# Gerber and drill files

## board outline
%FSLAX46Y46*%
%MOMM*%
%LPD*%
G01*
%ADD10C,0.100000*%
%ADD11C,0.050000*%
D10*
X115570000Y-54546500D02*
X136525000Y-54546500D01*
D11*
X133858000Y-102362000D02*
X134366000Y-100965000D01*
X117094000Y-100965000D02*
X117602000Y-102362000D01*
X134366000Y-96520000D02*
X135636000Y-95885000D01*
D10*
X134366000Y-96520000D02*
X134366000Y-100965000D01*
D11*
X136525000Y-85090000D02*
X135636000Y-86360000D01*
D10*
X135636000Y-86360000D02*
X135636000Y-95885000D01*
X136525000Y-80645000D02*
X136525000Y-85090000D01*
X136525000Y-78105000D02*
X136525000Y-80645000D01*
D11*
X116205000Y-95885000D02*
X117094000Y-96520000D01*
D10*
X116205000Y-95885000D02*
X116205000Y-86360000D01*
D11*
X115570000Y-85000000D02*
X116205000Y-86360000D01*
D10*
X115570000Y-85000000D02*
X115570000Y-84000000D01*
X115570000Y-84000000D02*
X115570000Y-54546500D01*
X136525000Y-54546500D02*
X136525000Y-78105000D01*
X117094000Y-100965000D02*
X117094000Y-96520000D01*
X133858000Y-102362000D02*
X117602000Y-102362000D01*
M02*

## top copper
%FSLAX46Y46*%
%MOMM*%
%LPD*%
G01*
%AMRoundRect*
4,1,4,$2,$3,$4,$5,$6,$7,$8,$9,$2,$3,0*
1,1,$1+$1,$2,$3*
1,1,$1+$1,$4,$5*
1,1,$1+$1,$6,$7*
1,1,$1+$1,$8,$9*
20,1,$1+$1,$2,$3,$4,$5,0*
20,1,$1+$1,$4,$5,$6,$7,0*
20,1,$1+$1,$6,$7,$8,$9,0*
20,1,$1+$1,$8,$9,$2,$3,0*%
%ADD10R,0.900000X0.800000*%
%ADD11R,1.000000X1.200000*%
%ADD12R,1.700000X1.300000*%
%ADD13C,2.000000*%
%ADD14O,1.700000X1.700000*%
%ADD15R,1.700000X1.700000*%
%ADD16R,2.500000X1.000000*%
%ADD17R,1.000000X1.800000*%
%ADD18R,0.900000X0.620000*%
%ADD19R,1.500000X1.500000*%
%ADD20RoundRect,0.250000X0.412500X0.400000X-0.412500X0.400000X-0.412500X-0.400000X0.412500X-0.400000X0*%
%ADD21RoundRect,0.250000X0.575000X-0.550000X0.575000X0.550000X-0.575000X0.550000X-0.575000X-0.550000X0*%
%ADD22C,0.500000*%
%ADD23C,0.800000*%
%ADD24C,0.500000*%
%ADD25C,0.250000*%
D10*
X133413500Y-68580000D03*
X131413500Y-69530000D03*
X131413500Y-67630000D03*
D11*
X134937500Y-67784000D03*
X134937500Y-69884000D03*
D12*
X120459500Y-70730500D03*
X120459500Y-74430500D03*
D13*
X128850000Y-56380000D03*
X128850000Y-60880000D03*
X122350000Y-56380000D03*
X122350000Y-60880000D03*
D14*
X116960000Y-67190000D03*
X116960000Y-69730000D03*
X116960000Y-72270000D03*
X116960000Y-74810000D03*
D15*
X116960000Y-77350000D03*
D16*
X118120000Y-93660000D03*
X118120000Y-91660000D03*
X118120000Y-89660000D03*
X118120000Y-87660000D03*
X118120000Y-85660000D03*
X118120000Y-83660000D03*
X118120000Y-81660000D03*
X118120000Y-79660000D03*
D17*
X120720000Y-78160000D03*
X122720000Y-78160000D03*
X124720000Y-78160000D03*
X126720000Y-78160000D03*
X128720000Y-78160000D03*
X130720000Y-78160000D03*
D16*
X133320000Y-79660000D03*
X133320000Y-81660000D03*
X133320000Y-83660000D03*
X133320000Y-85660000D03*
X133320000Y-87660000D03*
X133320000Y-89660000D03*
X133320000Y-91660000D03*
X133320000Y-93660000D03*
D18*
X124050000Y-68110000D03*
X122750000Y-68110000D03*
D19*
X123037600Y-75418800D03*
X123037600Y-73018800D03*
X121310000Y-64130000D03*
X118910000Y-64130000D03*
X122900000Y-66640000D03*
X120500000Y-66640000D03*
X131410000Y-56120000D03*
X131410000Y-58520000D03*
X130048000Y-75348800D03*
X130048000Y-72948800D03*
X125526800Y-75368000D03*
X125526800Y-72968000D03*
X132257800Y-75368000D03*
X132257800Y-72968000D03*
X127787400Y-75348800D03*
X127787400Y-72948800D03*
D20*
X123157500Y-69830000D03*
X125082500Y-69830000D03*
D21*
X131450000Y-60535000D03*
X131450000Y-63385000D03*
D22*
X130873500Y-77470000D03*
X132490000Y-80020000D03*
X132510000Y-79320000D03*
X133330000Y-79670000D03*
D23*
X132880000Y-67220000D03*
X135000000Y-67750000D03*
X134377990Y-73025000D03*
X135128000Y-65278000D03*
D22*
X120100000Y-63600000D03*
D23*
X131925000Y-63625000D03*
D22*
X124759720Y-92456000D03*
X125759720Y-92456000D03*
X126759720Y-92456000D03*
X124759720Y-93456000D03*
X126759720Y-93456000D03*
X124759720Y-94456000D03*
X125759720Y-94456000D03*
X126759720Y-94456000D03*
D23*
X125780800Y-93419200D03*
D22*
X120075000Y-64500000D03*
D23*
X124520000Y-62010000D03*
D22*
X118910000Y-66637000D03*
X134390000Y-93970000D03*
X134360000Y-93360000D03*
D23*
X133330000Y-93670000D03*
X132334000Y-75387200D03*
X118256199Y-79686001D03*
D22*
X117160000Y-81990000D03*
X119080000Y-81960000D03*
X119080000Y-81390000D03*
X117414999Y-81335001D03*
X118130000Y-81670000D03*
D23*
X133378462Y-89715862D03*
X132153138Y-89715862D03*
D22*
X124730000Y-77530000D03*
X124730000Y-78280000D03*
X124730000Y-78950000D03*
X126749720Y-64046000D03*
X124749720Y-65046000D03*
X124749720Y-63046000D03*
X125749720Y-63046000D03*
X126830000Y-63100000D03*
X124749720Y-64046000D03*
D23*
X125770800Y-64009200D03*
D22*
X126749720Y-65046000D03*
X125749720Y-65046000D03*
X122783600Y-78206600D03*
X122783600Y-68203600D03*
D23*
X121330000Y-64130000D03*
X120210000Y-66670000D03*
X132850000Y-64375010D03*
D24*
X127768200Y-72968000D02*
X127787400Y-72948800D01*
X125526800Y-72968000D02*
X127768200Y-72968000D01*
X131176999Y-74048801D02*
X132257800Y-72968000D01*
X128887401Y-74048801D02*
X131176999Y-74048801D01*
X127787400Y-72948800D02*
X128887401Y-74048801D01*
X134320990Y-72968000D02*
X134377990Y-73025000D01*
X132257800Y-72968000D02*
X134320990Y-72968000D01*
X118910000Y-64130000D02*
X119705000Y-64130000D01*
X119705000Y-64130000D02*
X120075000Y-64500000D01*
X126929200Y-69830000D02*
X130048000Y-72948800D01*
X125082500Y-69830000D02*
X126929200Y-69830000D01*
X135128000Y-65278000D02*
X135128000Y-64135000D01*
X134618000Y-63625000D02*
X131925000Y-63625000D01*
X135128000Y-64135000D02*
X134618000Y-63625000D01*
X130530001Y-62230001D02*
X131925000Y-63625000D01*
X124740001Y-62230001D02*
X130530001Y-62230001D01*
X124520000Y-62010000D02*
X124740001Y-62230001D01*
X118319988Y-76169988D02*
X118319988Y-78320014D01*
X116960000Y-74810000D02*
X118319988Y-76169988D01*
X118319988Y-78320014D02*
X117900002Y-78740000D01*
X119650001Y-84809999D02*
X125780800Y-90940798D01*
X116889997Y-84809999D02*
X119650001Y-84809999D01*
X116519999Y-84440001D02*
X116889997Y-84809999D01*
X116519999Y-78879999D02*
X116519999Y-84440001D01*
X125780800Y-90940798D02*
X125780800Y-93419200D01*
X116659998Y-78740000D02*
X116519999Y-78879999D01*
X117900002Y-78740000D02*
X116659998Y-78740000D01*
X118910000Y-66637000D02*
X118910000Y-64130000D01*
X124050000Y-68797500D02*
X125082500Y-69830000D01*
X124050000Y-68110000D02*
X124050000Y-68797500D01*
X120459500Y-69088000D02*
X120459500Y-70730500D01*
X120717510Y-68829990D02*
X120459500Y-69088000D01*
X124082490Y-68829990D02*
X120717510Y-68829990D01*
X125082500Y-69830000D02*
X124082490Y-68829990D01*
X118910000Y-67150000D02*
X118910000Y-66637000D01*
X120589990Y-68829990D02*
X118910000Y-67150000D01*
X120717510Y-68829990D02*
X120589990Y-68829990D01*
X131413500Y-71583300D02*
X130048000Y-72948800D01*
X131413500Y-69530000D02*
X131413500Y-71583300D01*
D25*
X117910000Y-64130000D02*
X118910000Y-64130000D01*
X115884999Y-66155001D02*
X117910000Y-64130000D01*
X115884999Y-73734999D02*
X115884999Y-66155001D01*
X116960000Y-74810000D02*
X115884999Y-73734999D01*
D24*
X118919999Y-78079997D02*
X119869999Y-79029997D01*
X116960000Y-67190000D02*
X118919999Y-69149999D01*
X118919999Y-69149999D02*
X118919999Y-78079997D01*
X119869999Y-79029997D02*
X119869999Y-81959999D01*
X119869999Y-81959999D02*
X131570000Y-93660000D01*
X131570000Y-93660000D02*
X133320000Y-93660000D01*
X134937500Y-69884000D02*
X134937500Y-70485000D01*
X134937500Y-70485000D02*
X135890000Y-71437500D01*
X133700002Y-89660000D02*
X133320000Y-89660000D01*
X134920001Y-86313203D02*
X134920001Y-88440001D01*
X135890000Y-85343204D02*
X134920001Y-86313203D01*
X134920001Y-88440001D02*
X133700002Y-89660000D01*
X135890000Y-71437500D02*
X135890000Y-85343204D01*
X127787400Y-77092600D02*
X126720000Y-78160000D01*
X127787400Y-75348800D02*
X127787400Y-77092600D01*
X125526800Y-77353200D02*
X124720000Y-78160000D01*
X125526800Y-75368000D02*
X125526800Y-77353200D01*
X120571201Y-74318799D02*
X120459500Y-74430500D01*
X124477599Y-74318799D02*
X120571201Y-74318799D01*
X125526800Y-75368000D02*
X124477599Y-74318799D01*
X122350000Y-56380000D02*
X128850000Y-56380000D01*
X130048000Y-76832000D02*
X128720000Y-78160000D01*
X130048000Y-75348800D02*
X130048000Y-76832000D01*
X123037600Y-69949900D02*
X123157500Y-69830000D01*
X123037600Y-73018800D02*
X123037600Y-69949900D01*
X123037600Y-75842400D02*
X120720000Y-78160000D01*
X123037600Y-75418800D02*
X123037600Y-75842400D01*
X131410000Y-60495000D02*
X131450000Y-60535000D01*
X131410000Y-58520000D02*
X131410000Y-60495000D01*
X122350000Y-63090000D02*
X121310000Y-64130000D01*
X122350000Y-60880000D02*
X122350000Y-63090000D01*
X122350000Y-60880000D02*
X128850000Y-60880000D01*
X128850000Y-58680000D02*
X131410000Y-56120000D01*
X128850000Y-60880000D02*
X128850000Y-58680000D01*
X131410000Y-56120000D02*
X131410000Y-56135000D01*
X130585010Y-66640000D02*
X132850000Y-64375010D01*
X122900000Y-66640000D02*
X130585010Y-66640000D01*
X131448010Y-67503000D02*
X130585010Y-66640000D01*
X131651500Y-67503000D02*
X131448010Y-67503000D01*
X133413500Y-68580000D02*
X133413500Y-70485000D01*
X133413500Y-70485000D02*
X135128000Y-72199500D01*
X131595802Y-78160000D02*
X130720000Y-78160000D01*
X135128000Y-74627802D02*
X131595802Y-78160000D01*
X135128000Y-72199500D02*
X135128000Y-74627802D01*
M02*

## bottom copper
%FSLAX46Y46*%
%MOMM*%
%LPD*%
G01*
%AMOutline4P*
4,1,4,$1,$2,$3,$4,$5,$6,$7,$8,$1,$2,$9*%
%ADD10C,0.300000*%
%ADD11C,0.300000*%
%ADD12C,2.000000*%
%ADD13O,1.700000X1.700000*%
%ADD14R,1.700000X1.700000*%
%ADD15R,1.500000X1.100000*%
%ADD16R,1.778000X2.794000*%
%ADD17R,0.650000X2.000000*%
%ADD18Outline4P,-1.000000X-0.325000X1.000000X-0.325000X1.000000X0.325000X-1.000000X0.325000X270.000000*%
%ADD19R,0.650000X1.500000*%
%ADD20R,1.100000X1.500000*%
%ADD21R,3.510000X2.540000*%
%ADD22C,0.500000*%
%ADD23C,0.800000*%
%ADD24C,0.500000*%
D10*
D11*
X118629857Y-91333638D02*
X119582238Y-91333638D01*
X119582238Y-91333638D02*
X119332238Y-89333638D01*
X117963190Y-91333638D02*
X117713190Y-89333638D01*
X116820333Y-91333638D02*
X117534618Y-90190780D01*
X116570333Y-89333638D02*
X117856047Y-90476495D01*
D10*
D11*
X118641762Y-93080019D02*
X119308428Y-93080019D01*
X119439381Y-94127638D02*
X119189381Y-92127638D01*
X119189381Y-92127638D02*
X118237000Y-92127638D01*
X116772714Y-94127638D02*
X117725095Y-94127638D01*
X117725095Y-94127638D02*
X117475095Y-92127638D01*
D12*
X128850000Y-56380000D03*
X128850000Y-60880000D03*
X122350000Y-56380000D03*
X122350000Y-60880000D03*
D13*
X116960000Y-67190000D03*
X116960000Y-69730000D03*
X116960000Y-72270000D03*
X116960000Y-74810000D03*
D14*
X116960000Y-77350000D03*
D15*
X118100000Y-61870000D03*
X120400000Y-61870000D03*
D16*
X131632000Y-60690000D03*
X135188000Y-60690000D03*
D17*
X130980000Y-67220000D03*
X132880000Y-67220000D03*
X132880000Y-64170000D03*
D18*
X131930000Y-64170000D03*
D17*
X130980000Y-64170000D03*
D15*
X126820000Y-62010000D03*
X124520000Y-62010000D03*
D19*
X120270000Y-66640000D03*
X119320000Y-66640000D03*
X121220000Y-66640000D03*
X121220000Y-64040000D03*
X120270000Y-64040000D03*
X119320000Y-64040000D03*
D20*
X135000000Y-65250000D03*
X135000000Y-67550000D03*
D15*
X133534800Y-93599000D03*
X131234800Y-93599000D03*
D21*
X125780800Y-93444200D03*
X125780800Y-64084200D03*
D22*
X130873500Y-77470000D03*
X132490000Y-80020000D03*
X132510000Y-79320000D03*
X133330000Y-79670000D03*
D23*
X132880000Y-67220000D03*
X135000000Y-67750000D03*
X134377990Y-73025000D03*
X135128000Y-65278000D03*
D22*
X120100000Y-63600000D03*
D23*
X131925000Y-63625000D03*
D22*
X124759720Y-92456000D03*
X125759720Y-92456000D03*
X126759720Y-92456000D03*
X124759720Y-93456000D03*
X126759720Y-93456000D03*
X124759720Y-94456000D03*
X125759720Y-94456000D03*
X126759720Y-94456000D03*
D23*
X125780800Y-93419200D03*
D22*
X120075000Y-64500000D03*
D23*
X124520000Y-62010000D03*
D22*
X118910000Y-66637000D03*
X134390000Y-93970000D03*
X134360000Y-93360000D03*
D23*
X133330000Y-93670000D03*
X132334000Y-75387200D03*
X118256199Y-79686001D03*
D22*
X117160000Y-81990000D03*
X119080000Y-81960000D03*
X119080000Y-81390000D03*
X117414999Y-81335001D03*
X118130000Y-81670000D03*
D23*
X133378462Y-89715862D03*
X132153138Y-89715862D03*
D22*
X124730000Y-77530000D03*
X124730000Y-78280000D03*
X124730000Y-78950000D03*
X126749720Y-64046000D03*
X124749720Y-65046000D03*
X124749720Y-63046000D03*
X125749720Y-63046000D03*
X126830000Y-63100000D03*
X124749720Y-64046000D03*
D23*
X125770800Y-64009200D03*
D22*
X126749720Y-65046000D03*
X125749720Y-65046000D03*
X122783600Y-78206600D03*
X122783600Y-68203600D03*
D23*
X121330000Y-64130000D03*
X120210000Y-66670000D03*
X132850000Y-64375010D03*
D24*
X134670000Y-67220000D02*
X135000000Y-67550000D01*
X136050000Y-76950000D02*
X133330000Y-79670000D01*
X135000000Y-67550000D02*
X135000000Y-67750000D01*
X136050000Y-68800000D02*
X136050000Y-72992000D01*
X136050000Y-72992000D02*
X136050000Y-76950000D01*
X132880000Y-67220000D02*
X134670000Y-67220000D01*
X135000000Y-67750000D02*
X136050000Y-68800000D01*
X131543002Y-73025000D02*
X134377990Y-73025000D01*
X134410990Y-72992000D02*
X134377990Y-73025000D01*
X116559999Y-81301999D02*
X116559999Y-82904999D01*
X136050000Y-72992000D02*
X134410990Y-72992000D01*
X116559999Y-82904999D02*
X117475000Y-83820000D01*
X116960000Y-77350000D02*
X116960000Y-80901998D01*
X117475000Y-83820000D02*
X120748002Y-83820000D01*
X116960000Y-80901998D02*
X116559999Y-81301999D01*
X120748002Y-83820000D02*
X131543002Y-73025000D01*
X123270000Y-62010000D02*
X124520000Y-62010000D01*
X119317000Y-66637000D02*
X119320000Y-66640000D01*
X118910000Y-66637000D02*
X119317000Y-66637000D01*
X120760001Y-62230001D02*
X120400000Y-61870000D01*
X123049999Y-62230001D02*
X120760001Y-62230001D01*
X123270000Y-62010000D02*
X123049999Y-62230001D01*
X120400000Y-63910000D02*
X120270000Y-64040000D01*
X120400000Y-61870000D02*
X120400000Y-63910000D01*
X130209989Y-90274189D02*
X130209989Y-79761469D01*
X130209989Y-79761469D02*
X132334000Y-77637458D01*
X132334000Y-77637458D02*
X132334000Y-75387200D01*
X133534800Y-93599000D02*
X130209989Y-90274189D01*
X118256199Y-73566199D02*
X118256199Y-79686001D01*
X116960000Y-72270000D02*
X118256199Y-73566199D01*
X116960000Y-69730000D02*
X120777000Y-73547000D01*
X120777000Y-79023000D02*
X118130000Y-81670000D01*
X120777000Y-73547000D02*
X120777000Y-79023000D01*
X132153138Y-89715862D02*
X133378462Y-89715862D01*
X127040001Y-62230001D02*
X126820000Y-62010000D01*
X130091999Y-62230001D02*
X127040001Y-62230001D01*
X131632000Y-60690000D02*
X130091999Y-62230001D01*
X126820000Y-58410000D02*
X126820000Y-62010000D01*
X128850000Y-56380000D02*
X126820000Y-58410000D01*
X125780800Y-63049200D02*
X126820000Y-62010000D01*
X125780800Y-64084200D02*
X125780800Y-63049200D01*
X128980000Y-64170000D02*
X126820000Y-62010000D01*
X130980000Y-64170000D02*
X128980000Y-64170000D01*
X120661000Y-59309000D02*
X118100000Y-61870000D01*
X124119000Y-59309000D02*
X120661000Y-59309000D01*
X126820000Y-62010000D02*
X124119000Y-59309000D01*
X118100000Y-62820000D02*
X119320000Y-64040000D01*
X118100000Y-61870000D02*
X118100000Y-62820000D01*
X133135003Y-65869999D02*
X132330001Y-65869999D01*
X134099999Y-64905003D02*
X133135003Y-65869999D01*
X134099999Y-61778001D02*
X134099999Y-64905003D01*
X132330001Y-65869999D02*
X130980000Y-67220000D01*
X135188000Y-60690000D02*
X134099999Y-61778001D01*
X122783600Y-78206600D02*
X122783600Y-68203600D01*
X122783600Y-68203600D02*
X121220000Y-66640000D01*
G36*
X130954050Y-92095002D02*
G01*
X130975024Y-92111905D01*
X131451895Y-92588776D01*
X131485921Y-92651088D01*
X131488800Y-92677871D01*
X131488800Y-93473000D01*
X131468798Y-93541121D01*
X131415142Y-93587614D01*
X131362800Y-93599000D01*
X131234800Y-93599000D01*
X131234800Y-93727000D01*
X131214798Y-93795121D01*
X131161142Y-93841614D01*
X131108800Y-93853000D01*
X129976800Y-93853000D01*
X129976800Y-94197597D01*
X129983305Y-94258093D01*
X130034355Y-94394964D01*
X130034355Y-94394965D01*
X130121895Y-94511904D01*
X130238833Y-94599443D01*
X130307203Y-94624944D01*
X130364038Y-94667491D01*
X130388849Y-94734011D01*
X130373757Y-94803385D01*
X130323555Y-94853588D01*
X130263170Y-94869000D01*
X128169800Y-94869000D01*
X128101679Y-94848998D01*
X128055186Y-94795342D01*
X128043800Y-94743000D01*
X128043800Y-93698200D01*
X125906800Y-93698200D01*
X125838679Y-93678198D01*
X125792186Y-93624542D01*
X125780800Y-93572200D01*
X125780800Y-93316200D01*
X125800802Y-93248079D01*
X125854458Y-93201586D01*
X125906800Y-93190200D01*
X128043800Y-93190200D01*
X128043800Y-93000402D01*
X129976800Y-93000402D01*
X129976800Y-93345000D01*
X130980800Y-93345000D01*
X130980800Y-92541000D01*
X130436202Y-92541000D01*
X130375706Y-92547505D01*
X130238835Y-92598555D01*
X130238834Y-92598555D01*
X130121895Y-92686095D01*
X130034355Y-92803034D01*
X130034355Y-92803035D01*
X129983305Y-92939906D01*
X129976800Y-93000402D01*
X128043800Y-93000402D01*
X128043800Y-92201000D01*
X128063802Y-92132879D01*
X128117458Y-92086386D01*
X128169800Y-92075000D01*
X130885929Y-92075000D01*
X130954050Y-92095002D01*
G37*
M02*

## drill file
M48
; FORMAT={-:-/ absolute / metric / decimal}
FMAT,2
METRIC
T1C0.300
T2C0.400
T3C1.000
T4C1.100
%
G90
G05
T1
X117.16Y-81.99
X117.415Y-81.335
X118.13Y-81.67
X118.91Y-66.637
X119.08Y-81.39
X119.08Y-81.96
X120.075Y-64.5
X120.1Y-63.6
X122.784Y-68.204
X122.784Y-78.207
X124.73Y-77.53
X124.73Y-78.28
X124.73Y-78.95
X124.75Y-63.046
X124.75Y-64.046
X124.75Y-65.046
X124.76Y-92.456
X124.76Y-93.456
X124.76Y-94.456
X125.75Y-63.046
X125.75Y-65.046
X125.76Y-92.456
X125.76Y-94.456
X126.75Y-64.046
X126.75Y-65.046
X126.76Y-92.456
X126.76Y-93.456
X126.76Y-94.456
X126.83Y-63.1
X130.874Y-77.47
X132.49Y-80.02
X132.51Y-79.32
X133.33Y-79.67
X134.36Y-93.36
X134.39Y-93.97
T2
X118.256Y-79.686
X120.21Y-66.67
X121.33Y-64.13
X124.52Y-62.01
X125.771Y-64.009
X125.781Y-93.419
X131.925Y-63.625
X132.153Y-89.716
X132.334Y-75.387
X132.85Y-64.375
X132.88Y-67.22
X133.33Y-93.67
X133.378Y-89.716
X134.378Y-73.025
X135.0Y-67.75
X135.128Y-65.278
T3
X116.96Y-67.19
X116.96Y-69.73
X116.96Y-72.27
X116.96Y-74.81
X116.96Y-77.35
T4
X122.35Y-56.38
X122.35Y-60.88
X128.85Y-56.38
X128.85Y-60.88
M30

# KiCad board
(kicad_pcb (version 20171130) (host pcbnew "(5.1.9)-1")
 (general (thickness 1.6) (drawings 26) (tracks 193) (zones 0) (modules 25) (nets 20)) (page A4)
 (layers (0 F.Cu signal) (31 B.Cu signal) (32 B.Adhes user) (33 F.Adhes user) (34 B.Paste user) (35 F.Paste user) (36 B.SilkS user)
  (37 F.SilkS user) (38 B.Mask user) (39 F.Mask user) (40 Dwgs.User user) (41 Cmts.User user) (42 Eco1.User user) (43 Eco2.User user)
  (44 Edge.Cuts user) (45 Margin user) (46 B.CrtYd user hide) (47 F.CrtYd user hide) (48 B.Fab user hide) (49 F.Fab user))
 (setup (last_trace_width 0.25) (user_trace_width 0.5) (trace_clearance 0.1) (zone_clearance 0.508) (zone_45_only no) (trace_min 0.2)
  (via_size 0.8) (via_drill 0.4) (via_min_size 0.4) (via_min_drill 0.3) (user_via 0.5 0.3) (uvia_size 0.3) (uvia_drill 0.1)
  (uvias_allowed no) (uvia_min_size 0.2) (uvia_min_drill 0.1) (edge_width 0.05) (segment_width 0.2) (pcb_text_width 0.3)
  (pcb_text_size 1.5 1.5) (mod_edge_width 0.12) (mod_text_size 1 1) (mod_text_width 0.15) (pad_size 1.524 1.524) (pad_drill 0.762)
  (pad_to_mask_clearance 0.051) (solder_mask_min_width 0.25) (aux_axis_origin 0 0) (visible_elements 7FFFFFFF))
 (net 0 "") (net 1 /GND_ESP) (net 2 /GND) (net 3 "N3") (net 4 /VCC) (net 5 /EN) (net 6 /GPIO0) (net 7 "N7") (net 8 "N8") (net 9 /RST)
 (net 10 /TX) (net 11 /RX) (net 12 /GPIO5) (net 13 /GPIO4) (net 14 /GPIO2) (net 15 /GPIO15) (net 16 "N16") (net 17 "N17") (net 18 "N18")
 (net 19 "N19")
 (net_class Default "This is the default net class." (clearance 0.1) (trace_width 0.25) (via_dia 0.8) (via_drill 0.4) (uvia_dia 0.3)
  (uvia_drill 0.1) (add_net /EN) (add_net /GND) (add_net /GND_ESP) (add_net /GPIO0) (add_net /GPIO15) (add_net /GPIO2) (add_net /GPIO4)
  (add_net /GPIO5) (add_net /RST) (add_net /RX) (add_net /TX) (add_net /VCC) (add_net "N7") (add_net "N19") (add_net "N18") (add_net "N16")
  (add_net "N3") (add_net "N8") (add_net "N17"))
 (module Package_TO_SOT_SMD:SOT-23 (layer F.Cu) (at 132.4135 68.58)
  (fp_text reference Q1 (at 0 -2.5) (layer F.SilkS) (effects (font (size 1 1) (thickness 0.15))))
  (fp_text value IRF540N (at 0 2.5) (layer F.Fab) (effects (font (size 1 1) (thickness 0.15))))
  (pad 3 smd rect (at 1 0) (size 0.9 0.8) (layers F.Cu F.Paste F.Mask) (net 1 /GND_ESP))
  (pad 2 smd rect (at -1 0.95) (size 0.9 0.8) (layers F.Cu F.Paste F.Mask) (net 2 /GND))
  (pad 1 smd rect (at -1 -0.95) (size 0.9 0.8) (layers F.Cu F.Paste F.Mask) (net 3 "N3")))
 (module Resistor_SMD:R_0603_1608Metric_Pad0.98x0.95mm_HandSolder (layer F.Cu) (at 134.9375 68.834 90)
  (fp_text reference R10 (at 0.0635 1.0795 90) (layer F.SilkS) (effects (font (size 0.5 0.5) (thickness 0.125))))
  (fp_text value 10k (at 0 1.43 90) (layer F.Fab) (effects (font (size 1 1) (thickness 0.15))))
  (pad 2 smd rect (at 1.05 0 90) (size 1.2 1) (layers F.Cu F.Paste F.Mask) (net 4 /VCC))
  (pad 1 smd rect (at -1.05 0 90) (size 1.2 1) (layers F.Cu F.Paste F.Mask) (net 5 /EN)))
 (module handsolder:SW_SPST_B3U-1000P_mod (layer F.Cu) (at 120.4595 72.5805 90)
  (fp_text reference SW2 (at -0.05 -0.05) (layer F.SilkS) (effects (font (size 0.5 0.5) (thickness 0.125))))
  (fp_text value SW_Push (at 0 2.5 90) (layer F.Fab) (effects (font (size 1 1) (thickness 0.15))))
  (pad 2 smd rect (at 1.85 0 90) (size 1.3 1.7) (layers F.Cu F.Paste F.Mask) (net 2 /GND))
  (pad 1 smd rect (at -1.85 0 90) (size 1.3 1.7) (layers F.Cu F.Paste F.Mask) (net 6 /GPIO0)))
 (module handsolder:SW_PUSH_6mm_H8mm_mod (layer F.Cu) (at 122.35 56.38)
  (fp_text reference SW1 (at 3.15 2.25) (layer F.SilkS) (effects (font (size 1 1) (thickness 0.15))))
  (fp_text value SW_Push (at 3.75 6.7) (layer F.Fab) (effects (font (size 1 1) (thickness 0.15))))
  (pad 1 thru_hole circle (at 6.5 0 90) (size 2 2) (drill 1.1) (layers *.Cu *.Mask) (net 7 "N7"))
  (pad 2 thru_hole circle (at 6.5 4.5 90) (size 2 2) (drill 1.1) (layers *.Cu *.Mask) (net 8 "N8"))
  (pad 1 thru_hole circle (at 0 0 90) (size 2 2) (drill 1.1) (layers *.Cu *.Mask) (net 7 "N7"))
  (pad 2 thru_hole circle (at 0 4.5 90) (size 2 2) (drill 1.1) (layers *.Cu *.Mask) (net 8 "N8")))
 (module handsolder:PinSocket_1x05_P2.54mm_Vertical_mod (layer F.Cu) (at 116.96 77.35 180)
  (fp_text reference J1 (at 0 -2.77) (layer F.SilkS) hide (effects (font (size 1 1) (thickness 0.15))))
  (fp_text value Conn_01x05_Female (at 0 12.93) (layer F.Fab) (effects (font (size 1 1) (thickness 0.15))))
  (pad 5 thru_hole oval (at 0 10.16 180) (size 1.7 1.7) (drill 1) (layers *.Cu *.Mask) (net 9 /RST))
  (pad 4 thru_hole oval (at 0 7.62 180) (size 1.7 1.7) (drill 1) (layers *.Cu *.Mask) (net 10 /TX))
  (pad 3 thru_hole oval (at 0 5.08 180) (size 1.7 1.7) (drill 1) (layers *.Cu *.Mask) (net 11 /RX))
  (pad 2 thru_hole oval (at 0 2.54 180) (size 1.7 1.7) (drill 1) (layers *.Cu *.Mask) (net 2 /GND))
  (pad 1 thru_hole rect (at 0 0 180) (size 1.7 1.7) (drill 1) (layers *.Cu *.Mask) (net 4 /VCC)))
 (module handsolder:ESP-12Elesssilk (layer F.Cu) (at 125.72 90.16 180)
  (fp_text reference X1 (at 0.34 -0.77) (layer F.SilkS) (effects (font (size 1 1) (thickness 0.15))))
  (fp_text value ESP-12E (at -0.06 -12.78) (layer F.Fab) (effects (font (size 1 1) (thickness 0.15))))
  (pad 22 smd rect (at 7.6 -3.5 180) (size 2.5 1) (layers F.Cu F.Paste F.Mask))
  (pad 21 smd rect (at 7.6 -1.5 180) (size 2.5 1) (layers F.Cu F.Paste F.Mask))
  (pad 20 smd rect (at 7.6 0.5 180) (size 2.5 1) (layers F.Cu F.Paste F.Mask))
  (pad 19 smd rect (at 7.6 2.5 180) (size 2.5 1) (layers F.Cu F.Paste F.Mask))
  (pad 18 smd rect (at 7.6 4.5 180) (size 2.5 1) (layers F.Cu F.Paste F.Mask))
  (pad 17 smd rect (at 7.6 6.5 180) (size 2.5 1) (layers F.Cu F.Paste F.Mask))
  (pad 16 smd rect (at 7.6 8.5 180) (size 2.5 1) (layers F.Cu F.Paste F.Mask) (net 10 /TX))
  (pad 15 smd rect (at 7.6 10.5 180) (size 2.5 1) (layers F.Cu F.Paste F.Mask) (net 11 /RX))
  (pad 14 smd rect (at 5 12 180) (size 1 1.8) (layers F.Cu F.Paste F.Mask) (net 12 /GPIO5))
  (pad 13 smd rect (at 3 12 180) (size 1 1.8) (layers F.Cu F.Paste F.Mask) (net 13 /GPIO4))
  (pad 12 smd rect (at 1 12 180) (size 1 1.8) (layers F.Cu F.Paste F.Mask) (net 6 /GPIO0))
  (pad 11 smd rect (at -1 12 180) (size 1 1.8) (layers F.Cu F.Paste F.Mask) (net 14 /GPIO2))
  (pad 10 smd rect (at -3 12 180) (size 1 1.8) (layers F.Cu F.Paste F.Mask) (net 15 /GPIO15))
  (pad 9 smd rect (at -5 12 180) (size 1 1.8) (layers F.Cu F.Paste F.Mask) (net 1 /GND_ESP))
  (pad 8 smd rect (at -7.6 10.5 180) (size 2.5 1) (layers F.Cu F.Paste F.Mask) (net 4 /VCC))
  (pad 7 smd rect (at -7.6 8.5 180) (size 2.5 1) (layers F.Cu F.Paste F.Mask))
  (pad 6 smd rect (at -7.6 6.5 180) (size 2.5 1) (layers F.Cu F.Paste F.Mask))
  (pad 5 smd rect (at -7.6 4.5 180) (size 2.5 1) (layers F.Cu F.Paste F.Mask))
  (pad 4 smd rect (at -7.6 2.5 180) (size 2.5 1) (layers F.Cu F.Paste F.Mask))
  (pad 3 smd rect (at -7.6 0.5 180) (size 2.5 1) (layers F.Cu F.Paste F.Mask) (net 5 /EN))
  (pad 2 smd rect (at -7.6 -1.5 180) (size 2.5 1) (layers F.Cu F.Paste F.Mask))
  (pad 1 smd rect (at -7.6 -3.5 180) (size 2.5 1) (layers F.Cu F.Paste F.Mask) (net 9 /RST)))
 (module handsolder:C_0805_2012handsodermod (layer B.Cu) (at 119.25 61.87 180)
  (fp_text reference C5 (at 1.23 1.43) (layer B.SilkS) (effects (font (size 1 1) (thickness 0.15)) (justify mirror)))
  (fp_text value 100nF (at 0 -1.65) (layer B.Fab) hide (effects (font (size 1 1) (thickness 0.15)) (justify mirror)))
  (pad 2 smd rect (at 1.15 0 180) (size 1.5 1.1) (layers B.Cu B.Paste B.Mask) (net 7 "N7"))
  (pad 1 smd rect (at -1.15 0 180) (size 1.5 1.1) (layers B.Cu B.Paste B.Mask) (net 2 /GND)))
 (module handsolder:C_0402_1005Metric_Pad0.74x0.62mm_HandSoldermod (layer F.Cu) (at 123.4 68.11)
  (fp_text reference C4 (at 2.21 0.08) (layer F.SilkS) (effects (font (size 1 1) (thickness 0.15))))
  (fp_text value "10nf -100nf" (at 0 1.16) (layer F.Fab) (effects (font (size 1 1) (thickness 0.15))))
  (pad 2 smd rect (at 0.65 0) (size 0.9 0.62) (layers F.Cu F.Paste F.Mask) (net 2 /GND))
  (pad 1 smd rect (at -0.65 0) (size 0.9 0.62) (layers F.Cu F.Paste F.Mask) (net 13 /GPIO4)))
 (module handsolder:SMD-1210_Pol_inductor (layer B.Cu) (at 133.41 60.69)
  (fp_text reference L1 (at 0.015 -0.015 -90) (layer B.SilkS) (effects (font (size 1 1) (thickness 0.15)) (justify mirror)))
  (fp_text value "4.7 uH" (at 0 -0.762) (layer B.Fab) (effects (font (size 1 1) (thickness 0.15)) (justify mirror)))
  (pad 1 smd rect (at -1.778 0) (size 1.778 2.794) (layers B.Cu B.Paste B.Mask) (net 7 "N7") (zone_connect 2))
  (pad 2 smd rect (at 1.778 0) (size 1.778 2.794) (layers B.Cu B.Paste B.Mask) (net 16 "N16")))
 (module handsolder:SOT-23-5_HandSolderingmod (layer B.Cu) (at 131.93 65.72 270)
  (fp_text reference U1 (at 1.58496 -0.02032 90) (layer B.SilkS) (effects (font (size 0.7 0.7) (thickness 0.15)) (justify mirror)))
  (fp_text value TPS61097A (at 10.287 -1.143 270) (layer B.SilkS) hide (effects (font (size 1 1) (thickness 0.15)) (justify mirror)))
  (pad 5 smd rect (at 1.5 0.95 270) (size 2 0.65) (layers B.Cu B.Paste B.Mask) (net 16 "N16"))
  (pad 4 smd rect (at 1.5 -0.95 270) (size 2 0.65) (layers B.Cu B.Paste B.Mask) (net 4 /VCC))
  (pad 3 smd rect (at -1.55 -0.95 270) (size 2 0.65) (layers B.Cu B.Paste B.Mask) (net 3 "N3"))
  (pad 2 smd trapezoid (at -1.55 0 270) (size 2 0.65) (layers B.Cu B.Paste B.Mask) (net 2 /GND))
  (pad 1 smd rect (at -1.55 0.95 270) (size 2 0.65) (layers B.Cu B.Paste B.Mask) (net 7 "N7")))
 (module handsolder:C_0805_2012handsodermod (layer B.Cu) (at 125.67 62.01)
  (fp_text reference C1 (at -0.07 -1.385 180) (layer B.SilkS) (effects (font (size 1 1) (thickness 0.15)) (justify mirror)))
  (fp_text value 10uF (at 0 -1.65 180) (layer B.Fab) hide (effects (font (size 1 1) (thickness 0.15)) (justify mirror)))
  (pad 2 smd rect (at 1.15 0) (size 1.5 1.1) (layers B.Cu B.Paste B.Mask) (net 7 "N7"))
  (pad 1 smd rect (at -1.15 0) (size 1.5 1.1) (layers B.Cu B.Paste B.Mask) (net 2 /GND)))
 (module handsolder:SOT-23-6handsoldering (layer B.Cu) (at 120.27 65.34 270)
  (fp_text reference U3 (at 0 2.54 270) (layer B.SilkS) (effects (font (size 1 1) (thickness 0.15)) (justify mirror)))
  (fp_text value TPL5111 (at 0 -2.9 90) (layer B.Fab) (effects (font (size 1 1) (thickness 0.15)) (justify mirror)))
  (pad 5 smd rect (at 1.3 0 270) (size 1.5 0.65) (layers B.Cu B.Paste B.Mask) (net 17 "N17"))
  (pad 6 smd rect (at 1.3 0.95 270) (size 1.5 0.65) (layers B.Cu B.Paste B.Mask) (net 2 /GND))
  (pad 4 smd rect (at 1.3 -0.95 270) (size 1.5 0.65) (layers B.Cu B.Paste B.Mask) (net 13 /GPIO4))
  (pad 3 smd rect (at -1.3 -0.95 270) (size 1.5 0.65) (layers B.Cu B.Paste B.Mask) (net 8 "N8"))
  (pad 2 smd rect (at -1.3 0 270) (size 1.5 0.65) (layers B.Cu B.Paste B.Mask) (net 2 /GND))
  (pad 1 smd rect (at -1.3 0.95 270) (size 1.5 0.65) (layers B.Cu B.Paste B.Mask) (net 7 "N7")))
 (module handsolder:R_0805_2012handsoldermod (layer F.Cu) (at 123.0376 74.2188 270)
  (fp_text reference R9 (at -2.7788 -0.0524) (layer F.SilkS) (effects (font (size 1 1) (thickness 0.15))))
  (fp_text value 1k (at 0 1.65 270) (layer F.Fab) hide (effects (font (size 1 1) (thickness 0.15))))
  (pad 2 smd rect (at 1.2 0 270) (size 1.5 1.5) (layers F.Cu F.Paste F.Mask) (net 12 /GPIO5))
  (pad 1 smd rect (at -1.2 0 270) (size 1.5 1.5) (layers F.Cu F.Paste F.Mask) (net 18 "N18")))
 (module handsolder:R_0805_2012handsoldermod (layer F.Cu) (at 120.11 64.13)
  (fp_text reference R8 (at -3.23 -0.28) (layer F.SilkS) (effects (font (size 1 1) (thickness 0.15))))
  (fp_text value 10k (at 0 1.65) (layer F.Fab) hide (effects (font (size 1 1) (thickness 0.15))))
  (pad 2 smd rect (at 1.2 0) (size 1.5 1.5) (layers F.Cu F.Paste F.Mask) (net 8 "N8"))
  (pad 1 smd rect (at -1.2 0) (size 1.5 1.5) (layers F.Cu F.Paste F.Mask) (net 2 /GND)))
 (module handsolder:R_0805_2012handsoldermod (layer F.Cu) (at 121.7 66.64)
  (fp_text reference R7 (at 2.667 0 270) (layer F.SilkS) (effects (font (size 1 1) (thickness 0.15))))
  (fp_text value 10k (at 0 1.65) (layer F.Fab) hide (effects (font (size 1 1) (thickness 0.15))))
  (pad 2 smd rect (at 1.2 0) (size 1.5 1.5) (layers F.Cu F.Paste F.Mask) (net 3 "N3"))
  (pad 1 smd rect (at -1.2 0) (size 1.5 1.5) (layers F.Cu F.Paste F.Mask) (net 17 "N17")))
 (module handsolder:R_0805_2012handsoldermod (layer F.Cu) (at 131.41 57.32 90)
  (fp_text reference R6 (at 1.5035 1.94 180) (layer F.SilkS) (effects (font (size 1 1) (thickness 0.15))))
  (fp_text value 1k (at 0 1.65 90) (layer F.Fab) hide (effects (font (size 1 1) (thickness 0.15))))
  (pad 2 smd rect (at 1.2 0 90) (size 1.5 1.5) (layers F.Cu F.Paste F.Mask) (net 8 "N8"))
  (pad 1 smd rect (at -1.2 0 90) (size 1.5 1.5) (layers F.Cu F.Paste F.Mask) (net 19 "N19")))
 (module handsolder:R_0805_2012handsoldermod (layer F.Cu) (at 130.048 74.1488 270)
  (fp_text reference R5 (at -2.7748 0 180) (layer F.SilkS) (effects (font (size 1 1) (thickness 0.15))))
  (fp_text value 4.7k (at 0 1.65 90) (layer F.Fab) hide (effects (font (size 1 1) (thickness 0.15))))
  (pad 2 smd rect (at 1.2 0 270) (size 1.5 1.5) (layers F.Cu F.Paste F.Mask) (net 15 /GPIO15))
  (pad 1 smd rect (at -1.2 0 270) (size 1.5 1.5) (layers F.Cu F.Paste F.Mask) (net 2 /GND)))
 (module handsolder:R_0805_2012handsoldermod (layer F.Cu) (at 125.5268 74.168 270)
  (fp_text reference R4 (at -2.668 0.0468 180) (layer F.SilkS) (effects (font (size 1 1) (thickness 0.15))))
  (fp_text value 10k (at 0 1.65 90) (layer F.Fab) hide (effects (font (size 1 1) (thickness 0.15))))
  (pad 2 smd rect (at 1.2 0 270) (size 1.5 1.5) (layers F.Cu F.Paste F.Mask) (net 6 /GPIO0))
  (pad 1 smd rect (at -1.2 0 270) (size 1.5 1.5) (layers F.Cu F.Paste F.Mask) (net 4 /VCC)))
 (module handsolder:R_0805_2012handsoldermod (layer F.Cu) (at 132.2578 74.168 270)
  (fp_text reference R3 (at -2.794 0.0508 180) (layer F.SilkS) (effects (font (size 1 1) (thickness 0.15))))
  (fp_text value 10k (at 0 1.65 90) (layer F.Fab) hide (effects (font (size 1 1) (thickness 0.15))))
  (pad 2 smd rect (at 1.2 0 270) (size 1.5 1.5) (layers F.Cu F.Paste F.Mask) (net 9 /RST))
  (pad 1 smd rect (at -1.2 0 270) (size 1.5 1.5) (layers F.Cu F.Paste F.Mask) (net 4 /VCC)))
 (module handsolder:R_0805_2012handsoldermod (layer F.Cu) (at 127.7874 74.1488 270)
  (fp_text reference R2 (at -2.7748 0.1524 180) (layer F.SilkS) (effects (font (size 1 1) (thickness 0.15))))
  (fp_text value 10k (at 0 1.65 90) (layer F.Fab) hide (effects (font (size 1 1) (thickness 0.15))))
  (pad 2 smd rect (at 1.2 0 270) (size 1.5 1.5) (layers F.Cu F.Paste F.Mask) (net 14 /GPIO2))
  (pad 1 smd rect (at -1.2 0 270) (size 1.5 1.5) (layers F.Cu F.Paste F.Mask) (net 4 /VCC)))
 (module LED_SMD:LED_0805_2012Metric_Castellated (layer F.Cu) (at 124.12 69.83 180)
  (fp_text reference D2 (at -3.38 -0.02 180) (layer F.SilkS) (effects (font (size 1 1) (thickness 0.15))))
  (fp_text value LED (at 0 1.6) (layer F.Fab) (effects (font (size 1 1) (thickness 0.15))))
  (pad 2 smd roundrect (at 0.9625 0 180) (size 1.325 1.3) (layers F.Cu F.Paste F.Mask) (roundrect_rratio 0.1923076923076923) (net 18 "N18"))
  (pad 1 smd roundrect (at -0.9625 0 180) (size 1.325 1.3) (layers F.Cu F.Paste F.Mask) (roundrect_rratio 0.1923076923076923) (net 2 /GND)))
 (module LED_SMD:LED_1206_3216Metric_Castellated (layer F.Cu) (at 131.45 61.96 90)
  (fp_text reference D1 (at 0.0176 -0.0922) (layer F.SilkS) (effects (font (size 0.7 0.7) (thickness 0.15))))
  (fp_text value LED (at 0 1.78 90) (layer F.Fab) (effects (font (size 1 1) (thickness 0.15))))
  (pad 2 smd roundrect (at 1.425 0 90) (size 1.6 1.65) (layers F.Cu F.Paste F.Mask) (roundrect_rratio 0.15625) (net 19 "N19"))
  (pad 1 smd roundrect (at -1.425 0 90) (size 1.6 1.65) (layers F.Cu F.Paste F.Mask) (roundrect_rratio 0.15625) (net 2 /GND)))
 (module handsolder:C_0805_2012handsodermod (layer B.Cu) (at 135 66.4 90)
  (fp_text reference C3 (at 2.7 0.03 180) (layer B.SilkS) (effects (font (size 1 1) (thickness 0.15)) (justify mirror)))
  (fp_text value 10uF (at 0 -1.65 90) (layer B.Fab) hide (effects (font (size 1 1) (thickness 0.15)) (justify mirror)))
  (pad 2 smd rect (at 1.15 0 90) (size 1.5 1.1) (layers B.Cu B.Paste B.Mask) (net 2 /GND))
  (pad 1 smd rect (at -1.15 0 90) (size 1.5 1.1) (layers B.Cu B.Paste B.Mask) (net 4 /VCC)))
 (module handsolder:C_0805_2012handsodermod (layer B.Cu) (at 132.3848 93.599)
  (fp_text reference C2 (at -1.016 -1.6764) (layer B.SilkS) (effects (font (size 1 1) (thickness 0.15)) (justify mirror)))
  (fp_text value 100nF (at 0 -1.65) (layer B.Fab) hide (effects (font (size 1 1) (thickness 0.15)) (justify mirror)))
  (pad 2 smd rect (at 1.15 0) (size 1.5 1.1) (layers B.Cu B.Paste B.Mask) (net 9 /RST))
  (pad 1 smd rect (at -1.15 0) (size 1.5 1.1) (layers B.Cu B.Paste B.Mask) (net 2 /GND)))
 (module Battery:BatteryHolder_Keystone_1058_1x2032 (layer B.Cu) (at 125.7808 78.7642 270)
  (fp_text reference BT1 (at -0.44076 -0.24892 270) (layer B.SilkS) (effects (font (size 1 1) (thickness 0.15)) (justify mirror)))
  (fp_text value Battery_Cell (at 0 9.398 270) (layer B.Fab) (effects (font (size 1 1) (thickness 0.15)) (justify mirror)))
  (pad 2 smd rect (at 14.68 0 270) (size 2.54 3.51) (layers B.Cu B.Paste B.Mask) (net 2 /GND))
  (pad 1 smd rect (at -14.68 0 270) (size 2.54 3.51) (layers B.Cu B.Paste B.Mask) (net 7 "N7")))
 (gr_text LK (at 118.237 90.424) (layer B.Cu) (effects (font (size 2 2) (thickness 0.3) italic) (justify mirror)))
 (gr_line (start 115.57 54.5465) (end 136.525 54.5465) (layer Edge.Cuts) (width 0.1))
 (gr_line (start 133.858 102.362) (end 134.366 100.965) (layer Edge.Cuts) (width 0.05))
 (gr_line (start 117.094 100.965) (end 117.602 102.362) (layer Edge.Cuts) (width 0.05))
 (gr_line (start 134.366 96.52) (end 135.636 95.885) (layer Edge.Cuts) (width 0.05))
 (gr_line (start 134.366 96.52) (end 134.366 100.965) (layer Edge.Cuts) (width 0.1))
 (gr_line (start 136.525 85.09) (end 135.636 86.36) (layer Edge.Cuts) (width 0.05))
 (gr_line (start 135.636 86.36) (end 135.636 95.885) (layer Edge.Cuts) (width 0.1))
 (gr_line (start 136.525 80.645) (end 136.525 85.09) (layer Edge.Cuts) (width 0.1))
 (gr_line (start 136.525 78.105) (end 136.525 80.645) (layer Edge.Cuts) (width 0.1))
 (gr_line (start 116.205 95.885) (end 117.094 96.52) (layer Edge.Cuts) (width 0.05))
 (gr_line (start 116.205 95.885) (end 116.205 86.36) (layer Edge.Cuts) (width 0.1))
 (gr_line (start 115.57 85) (end 116.205 86.36) (layer Edge.Cuts) (width 0.05))
 (gr_line (start 115.57 85) (end 115.57 84) (layer Edge.Cuts) (width 0.1))
 (gr_line (start 115.57 84) (end 115.57 54.5465) (layer Edge.Cuts) (width 0.1))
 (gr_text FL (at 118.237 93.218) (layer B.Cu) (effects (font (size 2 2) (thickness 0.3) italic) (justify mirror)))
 (gr_line (start 136.525 54.5465) (end 136.525 78.105) (layer Edge.Cuts) (width 0.1))
 (gr_line (start 117.094 100.965) (end 117.094 96.52) (layer Edge.Cuts) (width 0.1))
 (gr_line (start 133.858 102.362) (end 117.602 102.362) (layer Edge.Cuts) (width 0.1))
 (via (at 130.8735 77.47) (size 0.5) (drill 0.3) (layers F.Cu B.Cu) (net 1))
 (via (at 132.49 80.02) (size 0.5) (drill 0.3) (layers F.Cu B.Cu) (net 4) (status 30))
 (via (at 132.51 79.32) (size 0.5) (drill 0.3) (layers F.Cu B.Cu) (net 4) (status 30))
 (via (at 133.33 79.67) (size 0.5) (drill 0.3) (layers F.Cu B.Cu) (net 4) (status 30))
 (segment (start 127.7682 72.968) (end 127.7874 72.9488) (width 0.5) (layer F.Cu) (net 4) (status 30))
 (segment (start 125.5268 72.968) (end 127.7682 72.968) (width 0.5) (layer F.Cu) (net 4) (status 30))
 (segment (start 131.176999 74.048801) (end 132.2578 72.968) (width 0.5) (layer F.Cu) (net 4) (status 20))
 (segment (start 128.887401 74.048801) (end 131.176999 74.048801) (width 0.5) (layer F.Cu) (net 4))
 (segment (start 127.7874 72.9488) (end 128.887401 74.048801) (width 0.5) (layer F.Cu) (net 4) (status 10))
 (segment (start 134.67 67.22) (end 135 67.55) (width 0.5) (layer B.Cu) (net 4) (status 30))
 (segment (start 136.05 76.95) (end 133.33 79.67) (width 0.5) (layer B.Cu) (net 4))
 (segment (start 135 67.55) (end 135 67.75) (width 0.5) (layer B.Cu) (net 4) (status 30))
 (segment (start 136.05 68.8) (end 136.05 72.992) (width 0.5) (layer B.Cu) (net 4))
 (segment (start 136.05 72.992) (end 136.05 76.95) (width 0.5) (layer B.Cu) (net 4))
 (segment (start 132.88 67.22) (end 134.67 67.22) (width 0.5) (layer B.Cu) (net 4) (status 30))
 (via (at 132.88 67.22) (size 0.8) (drill 0.4) (layers F.Cu B.Cu) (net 4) (status 30))
 (segment (start 135 67.75) (end 136.05 68.8) (width 0.5) (layer B.Cu) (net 4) (status 10))
 (via (at 135 67.75) (size 0.8) (drill 0.4) (layers F.Cu B.Cu) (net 4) (status 30))
 (via (at 134.37799 73.025) (size 0.8) (drill 0.4) (layers F.Cu B.Cu) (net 4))
 (segment (start 131.543002 73.025) (end 134.37799 73.025) (width 0.5) (layer B.Cu) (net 4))
 (segment (start 134.41099 72.992) (end 134.37799 73.025) (width 0.5) (layer B.Cu) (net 4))
 (segment (start 134.32099 72.968) (end 134.37799 73.025) (width 0.5) (layer F.Cu) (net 4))
 (segment (start 132.2578 72.968) (end 134.32099 72.968) (width 0.5) (layer F.Cu) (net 4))
 (segment (start 116.559999 81.301999) (end 116.559999 82.904999) (width 0.5) (layer B.Cu) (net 4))
 (segment (start 136.05 72.992) (end 134.41099 72.992) (width 0.5) (layer B.Cu) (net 4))
 (segment (start 116.559999 82.904999) (end 117.475 83.82) (width 0.5) (layer B.Cu) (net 4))
 (segment (start 116.96 77.35) (end 116.96 80.901998) (width 0.5) (layer B.Cu) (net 4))
 (segment (start 117.475 83.82) (end 120.748002 83.82) (width 0.5) (layer B.Cu) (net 4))
 (segment (start 116.96 80.901998) (end 116.559999 81.301999) (width 0.5) (layer B.Cu) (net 4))
 (segment (start 120.748002 83.82) (end 131.543002 73.025) (width 0.5) (layer B.Cu) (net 4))
 (via (at 135.128 65.278) (size 0.8) (drill 0.4) (layers F.Cu B.Cu) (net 2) (status 30))
 (via (at 120.1 63.6) (size 0.5) (drill 0.3) (layers F.Cu B.Cu) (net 2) (status 30))
 (via (at 131.925 63.625) (size 0.8) (drill 0.4) (layers F.Cu B.Cu) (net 2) (status 30))
 (via (at 124.75972 92.456) (size 0.5) (drill 0.3) (layers F.Cu B.Cu) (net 2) (status 30))
 (via (at 125.75972 92.456) (size 0.5) (drill 0.3) (layers F.Cu B.Cu) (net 2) (status 30))
 (via (at 126.75972 92.456) (size 0.5) (drill 0.3) (layers F.Cu B.Cu) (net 2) (status 30))
 (via (at 124.75972 93.456) (size 0.5) (drill 0.3) (layers F.Cu B.Cu) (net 2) (status 30))
 (via (at 126.75972 93.456) (size 0.5) (drill 0.3) (layers F.Cu B.Cu) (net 2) (status 30))
 (via (at 124.75972 94.456) (size 0.5) (drill 0.3) (layers F.Cu B.Cu) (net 2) (status 30))
 (via (at 125.75972 94.456) (size 0.5) (drill 0.3) (layers F.Cu B.Cu) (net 2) (status 30))
 (via (at 126.75972 94.456) (size 0.5) (drill 0.3) (layers F.Cu B.Cu) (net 2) (status 30))
 (via (at 125.7808 93.4192) (size 0.8) (drill 0.4) (layers F.Cu B.Cu) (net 2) (status 30))
 (segment (start 118.91 64.13) (end 119.705 64.13) (width 0.5) (layer F.Cu) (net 2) (status 10))
 (segment (start 119.705 64.13) (end 120.075 64.5) (width 0.5) (layer F.Cu) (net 2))
 (via (at 120.075 64.5) (size 0.5) (drill 0.3) (layers F.Cu B.Cu) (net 2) (status 30))
 (segment (start 126.9292 69.83) (end 130.048 72.9488) (width 0.5) (layer F.Cu) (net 2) (status 20))
 (segment (start 125.0825 69.83) (end 126.9292 69.83) (width 0.5) (layer F.Cu) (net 2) (status 10))
 (segment (start 123.27 62.01) (end 124.52 62.01) (width 0.5) (layer B.Cu) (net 2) (status 20))
 (segment (start 135.128 65.278) (end 135.128 64.135) (width 0.5) (layer F.Cu) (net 2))
 (segment (start 134.618 63.625) (end 131.925 63.625) (width 0.5) (layer F.Cu) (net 2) (status 20))
 (segment (start 135.128 64.135) (end 134.618 63.625) (width 0.5) (layer F.Cu) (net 2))
 (via (at 124.52 62.01) (size 0.8) (drill 0.4) (layers F.Cu B.Cu) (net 2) (status 30))
 (segment (start 130.530001 62.230001) (end 131.925 63.625) (width 0.5) (layer F.Cu) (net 2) (status 20))
 (segment (start 124.740001 62.230001) (end 130.530001 62.230001) (width 0.5) (layer F.Cu) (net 2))
 (segment (start 124.52 62.01) (end 124.740001 62.230001) (width 0.5) (layer F.Cu) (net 2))
 (segment (start 118.319988 76.169988) (end 118.319988 78.320014) (width 0.5) (layer F.Cu) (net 2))
 (segment (start 116.96 74.81) (end 118.319988 76.169988) (width 0.5) (layer F.Cu) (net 2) (status 10))
 (segment (start 118.319988 78.320014) (end 117.900002 78.74) (width 0.5) (layer F.Cu) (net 2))
 (segment (start 119.650001 84.809999) (end 125.7808 90.940798) (width 0.5) (layer F.Cu) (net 2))
 (segment (start 116.889997 84.809999) (end 119.650001 84.809999) (width 0.5) (layer F.Cu) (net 2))
 (segment (start 116.519999 84.440001) (end 116.889997 84.809999) (width 0.5) (layer F.Cu) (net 2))
 (segment (start 116.519999 78.879999) (end 116.519999 84.440001) (width 0.5) (layer F.Cu) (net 2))
 (segment (start 125.7808 90.940798) (end 125.7808 93.4192) (width 0.5) (layer F.Cu) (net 2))
 (segment (start 116.659998 78.74) (end 116.519999 78.879999) (width 0.5) (layer F.Cu) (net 2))
 (segment (start 117.900002 78.74) (end 116.659998 78.74) (width 0.5) (layer F.Cu) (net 2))
 (segment (start 118.91 66.637) (end 118.91 64.13) (width 0.5) (layer F.Cu) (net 2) (status 20))
 (via (at 118.91 66.637) (size 0.5) (drill 0.3) (layers F.Cu B.Cu) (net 2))
 (segment (start 119.317 66.637) (end 119.32 66.64) (width 0.5) (layer B.Cu) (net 2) (status 30))
 (segment (start 118.91 66.637) (end 119.317 66.637) (width 0.5) (layer B.Cu) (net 2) (status 20))
 (segment (start 124.05 68.7975) (end 125.0825 69.83) (width 0.5) (layer F.Cu) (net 2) (status 20))
 (segment (start 124.05 68.11) (end 124.05 68.7975) (width 0.5) (layer F.Cu) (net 2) (status 10))
 (segment (start 120.760001 62.230001) (end 120.4 61.87) (width 0.5) (layer B.Cu) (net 2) (status 30))
 (segment (start 123.049999 62.230001) (end 120.760001 62.230001) (width 0.5) (layer B.Cu) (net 2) (status 20))
 (segment (start 123.27 62.01) (end 123.049999 62.230001) (width 0.5) (layer B.Cu) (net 2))
 (segment (start 120.4 63.91) (end 120.27 64.04) (width 0.5) (layer B.Cu) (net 2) (status 30))
 (segment (start 120.4 61.87) (end 120.4 63.91) (width 0.5) (layer B.Cu) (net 2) (status 30))
 (segment (start 120.4595 69.088) (end 120.4595 70.7305) (width 0.5) (layer F.Cu) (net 2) (status 20))
 (segment (start 120.71751 68.82999) (end 120.4595 69.088) (width 0.5) (layer F.Cu) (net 2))
 (segment (start 124.08249 68.82999) (end 120.71751 68.82999) (width 0.5) (layer F.Cu) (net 2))
 (segment (start 125.0825 69.83) (end 124.08249 68.82999) (width 0.5) (layer F.Cu) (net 2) (status 10))
 (segment (start 118.91 67.15) (end 118.91 66.637) (width 0.5) (layer F.Cu) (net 2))
 (segment (start 120.58999 68.82999) (end 118.91 67.15) (width 0.5) (layer F.Cu) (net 2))
 (segment (start 120.71751 68.82999) (end 120.58999 68.82999) (width 0.5) (layer F.Cu) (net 2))
 (segment (start 131.4135 71.5833) (end 130.048 72.9488) (width 0.5) (layer F.Cu) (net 2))
 (segment (start 131.4135 69.53) (end 131.4135 71.5833) (width 0.5) (layer F.Cu) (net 2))
 (segment (start 117.91 64.13) (end 118.91 64.13) (width 0.25) (layer F.Cu) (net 2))
 (segment (start 115.884999 66.155001) (end 117.91 64.13) (width 0.25) (layer F.Cu) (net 2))
 (segment (start 115.884999 73.734999) (end 115.884999 66.155001) (width 0.25) (layer F.Cu) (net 2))
 (segment (start 116.96 74.81) (end 115.884999 73.734999) (width 0.25) (layer F.Cu) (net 2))
 (via (at 134.39 93.97) (size 0.5) (drill 0.3) (layers F.Cu B.Cu) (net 9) (status 30))
 (via (at 134.36 93.36) (size 0.5) (drill 0.3) (layers F.Cu B.Cu) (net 9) (status 30))
 (via (at 133.33 93.67) (size 0.8) (drill 0.4) (layers F.Cu B.Cu) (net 9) (status 30))
 (via (at 132.334 75.3872) (size 0.8) (drill 0.4) (layers F.Cu B.Cu) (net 9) (status 30))
 (segment (start 130.209989 90.274189) (end 130.209989 79.761469) (width 0.5) (layer B.Cu) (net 9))
 (segment (start 130.209989 79.761469) (end 132.334 77.637458) (width 0.5) (layer B.Cu) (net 9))
 (segment (start 132.334 77.637458) (end 132.334 75.3872) (width 0.5) (layer B.Cu) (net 9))
 (segment (start 133.5348 93.599) (end 130.209989 90.274189) (width 0.5) (layer B.Cu) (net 9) (status 10))
 (segment (start 118.919999 78.079997) (end 119.869999 79.029997) (width 0.5) (layer F.Cu) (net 9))
 (segment (start 116.96 67.19) (end 118.919999 69.149999) (width 0.5) (layer F.Cu) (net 9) (status 10))
 (segment (start 118.919999 69.149999) (end 118.919999 78.079997) (width 0.5) (layer F.Cu) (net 9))
 (segment (start 119.869999 79.029997) (end 119.869999 81.959999) (width 0.5) (layer F.Cu) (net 9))
 (segment (start 119.869999 81.959999) (end 131.57 93.66) (width 0.5) (layer F.Cu) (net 9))
 (segment (start 131.57 93.66) (end 133.32 93.66) (width 0.5) (layer F.Cu) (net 9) (status 20))
 (via (at 118.256199 79.686001) (size 0.8) (drill 0.4) (layers F.Cu B.Cu) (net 11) (status 30))
 (segment (start 118.256199 73.566199) (end 118.256199 79.686001) (width 0.5) (layer B.Cu) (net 11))
 (segment (start 116.96 72.27) (end 118.256199 73.566199) (width 0.5) (layer B.Cu) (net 11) (status 10))
 (via (at 117.16 81.99) (size 0.5) (drill 0.3) (layers F.Cu B.Cu) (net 10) (status 30))
 (via (at 119.08 81.96) (size 0.5) (drill 0.3) (layers F.Cu B.Cu) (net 10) (status 30))
 (via (at 119.08 81.39) (size 0.5) (drill 0.3) (layers F.Cu B.Cu) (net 10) (status 30))
 (via (at 117.414999 81.335001) (size 0.5) (drill 0.3) (layers F.Cu B.Cu) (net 10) (status 30))
 (via (at 118.13 81.67) (size 0.5) (drill 0.3) (layers F.Cu B.Cu) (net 10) (status 30))
 (segment (start 116.96 69.73) (end 120.777 73.547) (width 0.5) (layer B.Cu) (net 10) (status 10))
 (segment (start 120.777 79.023) (end 118.13 81.67) (width 0.5) (layer B.Cu) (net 10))
 (segment (start 120.777 73.547) (end 120.777 79.023) (width 0.5) (layer B.Cu) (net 10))
 (via (at 133.378462 89.715862) (size 0.8) (drill 0.4) (layers F.Cu B.Cu) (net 5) (status 30))
 (segment (start 132.153138 89.715862) (end 133.378462 89.715862) (width 0.5) (layer B.Cu) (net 5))
 (via (at 132.153138 89.715862) (size 0.8) (drill 0.4) (layers F.Cu B.Cu) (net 5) (status 30))
 (segment (start 134.9375 69.884) (end 134.9375 70.485) (width 0.5) (layer F.Cu) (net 5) (status 10))
 (segment (start 134.9375 70.485) (end 135.89 71.4375) (width 0.5) (layer F.Cu) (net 5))
 (segment (start 133.700002 89.66) (end 133.32 89.66) (width 0.5) (layer F.Cu) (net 5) (status 30))
 (segment (start 134.920001 86.313203) (end 134.920001 88.440001) (width 0.5) (layer F.Cu) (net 5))
 (segment (start 135.89 85.343204) (end 134.920001 86.313203) (width 0.5) (layer F.Cu) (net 5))
 (segment (start 134.920001 88.440001) (end 133.700002 89.66) (width 0.5) (layer F.Cu) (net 5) (status 20))
 (segment (start 135.89 71.4375) (end 135.89 85.343204) (width 0.5) (layer F.Cu) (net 5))
 (segment (start 127.7874 77.0926) (end 126.72 78.16) (width 0.5) (layer F.Cu) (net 14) (status 20))
 (segment (start 127.7874 75.3488) (end 127.7874 77.0926) (width 0.5) (layer F.Cu) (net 14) (status 10))
 (via (at 124.73 77.53) (size 0.5) (drill 0.3) (layers F.Cu B.Cu) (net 6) (status 30))
 (via (at 124.73 78.28) (size 0.5) (drill 0.3) (layers F.Cu B.Cu) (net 6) (status 30))
 (via (at 124.73 78.95) (size 0.5) (drill 0.3) (layers F.Cu B.Cu) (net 6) (status 30))
 (segment (start 125.5268 77.3532) (end 124.72 78.16) (width 0.5) (layer F.Cu) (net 6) (status 20))
 (segment (start 125.5268 75.368) (end 125.5268 77.3532) (width 0.5) (layer F.Cu) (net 6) (status 10))
 (segment (start 120.571201 74.318799) (end 120.4595 74.4305) (width 0.5) (layer F.Cu) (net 6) (status 30))
 (segment (start 124.477599 74.318799) (end 120.571201 74.318799) (width 0.5) (layer F.Cu) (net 6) (status 20))
 (segment (start 125.5268 75.368) (end 124.477599 74.318799) (width 0.5) (layer F.Cu) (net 6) (status 10))
 (via (at 126.74972 64.046) (size 0.5) (drill 0.3) (layers F.Cu B.Cu) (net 7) (status 30))
 (via (at 124.74972 65.046) (size 0.5) (drill 0.3) (layers F.Cu B.Cu) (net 7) (status 30))
 (via (at 124.74972 63.046) (size 0.5) (drill 0.3) (layers F.Cu B.Cu) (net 7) (status 30))
 (via (at 125.74972 63.046) (size 0.5) (drill 0.3) (layers F.Cu B.Cu) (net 7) (status 30))
 (via (at 126.83 63.1) (size 0.5) (drill 0.3) (layers F.Cu B.Cu) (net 7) (status 30))
 (via (at 124.74972 64.046) (size 0.5) (drill 0.3) (layers F.Cu B.Cu) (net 7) (status 30))
 (via (at 125.7708 64.0092) (size 0.8) (drill 0.4) (layers F.Cu B.Cu) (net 7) (status 30))
 (via (at 126.74972 65.046) (size 0.5) (drill 0.3) (layers F.Cu B.Cu) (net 7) (status 30))
 (via (at 125.74972 65.046) (size 0.5) (drill 0.3) (layers F.Cu B.Cu) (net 7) (status 30))
 (segment (start 122.35 56.38) (end 128.85 56.38) (width 0.5) (layer F.Cu) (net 7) (status 30))
 (segment (start 127.040001 62.230001) (end 126.82 62.01) (width 0.5) (layer B.Cu) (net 7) (status 30))
 (segment (start 130.091999 62.230001) (end 127.040001 62.230001) (width 0.5) (layer B.Cu) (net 7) (status 20))
 (segment (start 131.632 60.69) (end 130.091999 62.230001) (width 0.5) (layer B.Cu) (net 7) (status 10))
 (segment (start 126.82 58.41) (end 126.82 62.01) (width 0.5) (layer B.Cu) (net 7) (status 20))
 (segment (start 128.85 56.38) (end 126.82 58.41) (width 0.5) (layer B.Cu) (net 7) (status 10))
 (segment (start 125.7808 63.0492) (end 126.82 62.01) (width 0.5) (layer B.Cu) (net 7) (status 30))
 (segment (start 125.7808 64.0842) (end 125.7808 63.0492) (width 0.5) (layer B.Cu) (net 7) (status 30))
 (segment (start 128.98 64.17) (end 126.82 62.01) (width 0.5) (layer B.Cu) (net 7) (status 20))
 (segment (start 130.98 64.17) (end 128.98 64.17) (width 0.5) (layer B.Cu) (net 7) (status 10))
 (segment (start 120.661 59.309) (end 118.1 61.87) (width 0.5) (layer B.Cu) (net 7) (status 20))
 (segment (start 124.119 59.309) (end 120.661 59.309) (width 0.5) (layer B.Cu) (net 7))
 (segment (start 126.82 62.01) (end 124.119 59.309) (width 0.5) (layer B.Cu) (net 7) (status 10))
 (segment (start 118.1 62.82) (end 119.32 64.04) (width 0.5) (layer B.Cu) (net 7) (status 20))
 (segment (start 118.1 61.87) (end 118.1 62.82) (width 0.5) (layer B.Cu) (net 7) (status 10))
 (segment (start 133.135003 65.869999) (end 132.330001 65.869999) (width 0.5) (layer B.Cu) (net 16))
 (segment (start 134.099999 64.905003) (end 133.135003 65.869999) (width 0.5) (layer B.Cu) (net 16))
 (segment (start 134.099999 61.778001) (end 134.099999 64.905003) (width 0.5) (layer B.Cu) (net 16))
 (segment (start 132.330001 65.869999) (end 130.98 67.22) (width 0.5) (layer B.Cu) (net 16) (status 20))
 (segment (start 135.188 60.69) (end 134.099999 61.778001) (width 0.5) (layer B.Cu) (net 16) (status 10))
 (segment (start 130.048 76.832) (end 128.72 78.16) (width 0.5) (layer F.Cu) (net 15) (status 20))
 (segment (start 130.048 75.3488) (end 130.048 76.832) (width 0.5) (layer F.Cu) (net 15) (status 10))
 (via (at 122.7836 78.2066) (size 0.5) (drill 0.3) (layers F.Cu B.Cu) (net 13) (status 30))
 (segment (start 122.7836 78.2066) (end 122.7836 68.2036) (width 0.5) (layer B.Cu) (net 13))
 (segment (start 122.7836 68.2036) (end 121.22 66.64) (width 0.5) (layer B.Cu) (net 13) (status 20))
 (via (at 122.7836 68.2036) (size 0.5) (drill 0.3) (layers F.Cu B.Cu) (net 13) (status 30))
 (segment (start 123.0376 69.9499) (end 123.1575 69.83) (width 0.5) (layer F.Cu) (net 18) (status 30))
 (segment (start 123.0376 73.0188) (end 123.0376 69.9499) (width 0.5) (layer F.Cu) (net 18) (status 30))
 (segment (start 123.0376 75.8424) (end 120.72 78.16) (width 0.5) (layer F.Cu) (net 12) (status 30))
 (segment (start 123.0376 75.4188) (end 123.0376 75.8424) (width 0.5) (layer F.Cu) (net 12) (status 30))
 (segment (start 131.41 60.495) (end 131.45 60.535) (width 0.5) (layer F.Cu) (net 19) (status 30))
 (segment (start 131.41 58.52) (end 131.41 60.495) (width 0.5) (layer F.Cu) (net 19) (status 30))
 (via (at 121.33 64.13) (size 0.8) (drill 0.4) (layers F.Cu B.Cu) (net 8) (status 30))
 (segment (start 122.35 63.09) (end 121.31 64.13) (width 0.5) (layer F.Cu) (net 8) (status 20))
 (segment (start 122.35 60.88) (end 122.35 63.09) (width 0.5) (layer F.Cu) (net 8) (status 10))
 (segment (start 122.35 60.88) (end 128.85 60.88) (width 0.5) (layer F.Cu) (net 8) (status 30))
 (segment (start 128.85 58.68) (end 131.41 56.12) (width 0.5) (layer F.Cu) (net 8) (status 20))
 (segment (start 128.85 60.88) (end 128.85 58.68) (width 0.5) (layer F.Cu) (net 8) (status 10))
 (segment (start 131.41 56.12) (end 131.41 56.135) (width 0.5) (layer F.Cu) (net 8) (status 30))
 (via (at 120.21 66.67) (size 0.8) (drill 0.4) (layers F.Cu B.Cu) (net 17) (status 30))
 (segment (start 130.58501 66.64) (end 132.85 64.37501) (width 0.5) (layer F.Cu) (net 3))
 (via (at 132.85 64.37501) (size 0.8) (drill 0.4) (layers F.Cu B.Cu) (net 3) (status 30))
 (segment (start 122.9 66.64) (end 130.58501 66.64) (width 0.5) (layer F.Cu) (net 3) (status 10))
 (segment (start 131.44801 67.503) (end 130.58501 66.64) (width 0.5) (layer F.Cu) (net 3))
 (segment (start 131.6515 67.503) (end 131.44801 67.503) (width 0.5) (layer F.Cu) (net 3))
 (segment (start 133.4135 68.58) (end 133.4135 70.485) (width 0.5) (layer F.Cu) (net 1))
 (segment (start 133.4135 70.485) (end 135.128 72.1995) (width 0.5) (layer F.Cu) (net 1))
 (segment (start 131.595802 78.16) (end 130.72 78.16) (width 0.5) (layer F.Cu) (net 1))
 (segment (start 135.128 74.627802) (end 131.595802 78.16) (width 0.5) (layer F.Cu) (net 1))
 (segment (start 135.128 72.1995) (end 135.128 74.627802) (width 0.5) (layer F.Cu) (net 1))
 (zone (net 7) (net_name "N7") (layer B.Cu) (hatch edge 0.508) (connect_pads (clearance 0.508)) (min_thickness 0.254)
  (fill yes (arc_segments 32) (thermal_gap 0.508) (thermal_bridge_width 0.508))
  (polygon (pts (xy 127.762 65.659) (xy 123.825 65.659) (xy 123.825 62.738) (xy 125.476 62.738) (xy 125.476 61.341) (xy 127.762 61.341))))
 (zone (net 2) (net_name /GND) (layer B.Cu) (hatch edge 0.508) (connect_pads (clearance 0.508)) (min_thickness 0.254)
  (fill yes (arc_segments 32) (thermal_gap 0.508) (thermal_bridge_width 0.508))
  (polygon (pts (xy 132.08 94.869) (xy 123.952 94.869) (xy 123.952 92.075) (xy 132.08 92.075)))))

